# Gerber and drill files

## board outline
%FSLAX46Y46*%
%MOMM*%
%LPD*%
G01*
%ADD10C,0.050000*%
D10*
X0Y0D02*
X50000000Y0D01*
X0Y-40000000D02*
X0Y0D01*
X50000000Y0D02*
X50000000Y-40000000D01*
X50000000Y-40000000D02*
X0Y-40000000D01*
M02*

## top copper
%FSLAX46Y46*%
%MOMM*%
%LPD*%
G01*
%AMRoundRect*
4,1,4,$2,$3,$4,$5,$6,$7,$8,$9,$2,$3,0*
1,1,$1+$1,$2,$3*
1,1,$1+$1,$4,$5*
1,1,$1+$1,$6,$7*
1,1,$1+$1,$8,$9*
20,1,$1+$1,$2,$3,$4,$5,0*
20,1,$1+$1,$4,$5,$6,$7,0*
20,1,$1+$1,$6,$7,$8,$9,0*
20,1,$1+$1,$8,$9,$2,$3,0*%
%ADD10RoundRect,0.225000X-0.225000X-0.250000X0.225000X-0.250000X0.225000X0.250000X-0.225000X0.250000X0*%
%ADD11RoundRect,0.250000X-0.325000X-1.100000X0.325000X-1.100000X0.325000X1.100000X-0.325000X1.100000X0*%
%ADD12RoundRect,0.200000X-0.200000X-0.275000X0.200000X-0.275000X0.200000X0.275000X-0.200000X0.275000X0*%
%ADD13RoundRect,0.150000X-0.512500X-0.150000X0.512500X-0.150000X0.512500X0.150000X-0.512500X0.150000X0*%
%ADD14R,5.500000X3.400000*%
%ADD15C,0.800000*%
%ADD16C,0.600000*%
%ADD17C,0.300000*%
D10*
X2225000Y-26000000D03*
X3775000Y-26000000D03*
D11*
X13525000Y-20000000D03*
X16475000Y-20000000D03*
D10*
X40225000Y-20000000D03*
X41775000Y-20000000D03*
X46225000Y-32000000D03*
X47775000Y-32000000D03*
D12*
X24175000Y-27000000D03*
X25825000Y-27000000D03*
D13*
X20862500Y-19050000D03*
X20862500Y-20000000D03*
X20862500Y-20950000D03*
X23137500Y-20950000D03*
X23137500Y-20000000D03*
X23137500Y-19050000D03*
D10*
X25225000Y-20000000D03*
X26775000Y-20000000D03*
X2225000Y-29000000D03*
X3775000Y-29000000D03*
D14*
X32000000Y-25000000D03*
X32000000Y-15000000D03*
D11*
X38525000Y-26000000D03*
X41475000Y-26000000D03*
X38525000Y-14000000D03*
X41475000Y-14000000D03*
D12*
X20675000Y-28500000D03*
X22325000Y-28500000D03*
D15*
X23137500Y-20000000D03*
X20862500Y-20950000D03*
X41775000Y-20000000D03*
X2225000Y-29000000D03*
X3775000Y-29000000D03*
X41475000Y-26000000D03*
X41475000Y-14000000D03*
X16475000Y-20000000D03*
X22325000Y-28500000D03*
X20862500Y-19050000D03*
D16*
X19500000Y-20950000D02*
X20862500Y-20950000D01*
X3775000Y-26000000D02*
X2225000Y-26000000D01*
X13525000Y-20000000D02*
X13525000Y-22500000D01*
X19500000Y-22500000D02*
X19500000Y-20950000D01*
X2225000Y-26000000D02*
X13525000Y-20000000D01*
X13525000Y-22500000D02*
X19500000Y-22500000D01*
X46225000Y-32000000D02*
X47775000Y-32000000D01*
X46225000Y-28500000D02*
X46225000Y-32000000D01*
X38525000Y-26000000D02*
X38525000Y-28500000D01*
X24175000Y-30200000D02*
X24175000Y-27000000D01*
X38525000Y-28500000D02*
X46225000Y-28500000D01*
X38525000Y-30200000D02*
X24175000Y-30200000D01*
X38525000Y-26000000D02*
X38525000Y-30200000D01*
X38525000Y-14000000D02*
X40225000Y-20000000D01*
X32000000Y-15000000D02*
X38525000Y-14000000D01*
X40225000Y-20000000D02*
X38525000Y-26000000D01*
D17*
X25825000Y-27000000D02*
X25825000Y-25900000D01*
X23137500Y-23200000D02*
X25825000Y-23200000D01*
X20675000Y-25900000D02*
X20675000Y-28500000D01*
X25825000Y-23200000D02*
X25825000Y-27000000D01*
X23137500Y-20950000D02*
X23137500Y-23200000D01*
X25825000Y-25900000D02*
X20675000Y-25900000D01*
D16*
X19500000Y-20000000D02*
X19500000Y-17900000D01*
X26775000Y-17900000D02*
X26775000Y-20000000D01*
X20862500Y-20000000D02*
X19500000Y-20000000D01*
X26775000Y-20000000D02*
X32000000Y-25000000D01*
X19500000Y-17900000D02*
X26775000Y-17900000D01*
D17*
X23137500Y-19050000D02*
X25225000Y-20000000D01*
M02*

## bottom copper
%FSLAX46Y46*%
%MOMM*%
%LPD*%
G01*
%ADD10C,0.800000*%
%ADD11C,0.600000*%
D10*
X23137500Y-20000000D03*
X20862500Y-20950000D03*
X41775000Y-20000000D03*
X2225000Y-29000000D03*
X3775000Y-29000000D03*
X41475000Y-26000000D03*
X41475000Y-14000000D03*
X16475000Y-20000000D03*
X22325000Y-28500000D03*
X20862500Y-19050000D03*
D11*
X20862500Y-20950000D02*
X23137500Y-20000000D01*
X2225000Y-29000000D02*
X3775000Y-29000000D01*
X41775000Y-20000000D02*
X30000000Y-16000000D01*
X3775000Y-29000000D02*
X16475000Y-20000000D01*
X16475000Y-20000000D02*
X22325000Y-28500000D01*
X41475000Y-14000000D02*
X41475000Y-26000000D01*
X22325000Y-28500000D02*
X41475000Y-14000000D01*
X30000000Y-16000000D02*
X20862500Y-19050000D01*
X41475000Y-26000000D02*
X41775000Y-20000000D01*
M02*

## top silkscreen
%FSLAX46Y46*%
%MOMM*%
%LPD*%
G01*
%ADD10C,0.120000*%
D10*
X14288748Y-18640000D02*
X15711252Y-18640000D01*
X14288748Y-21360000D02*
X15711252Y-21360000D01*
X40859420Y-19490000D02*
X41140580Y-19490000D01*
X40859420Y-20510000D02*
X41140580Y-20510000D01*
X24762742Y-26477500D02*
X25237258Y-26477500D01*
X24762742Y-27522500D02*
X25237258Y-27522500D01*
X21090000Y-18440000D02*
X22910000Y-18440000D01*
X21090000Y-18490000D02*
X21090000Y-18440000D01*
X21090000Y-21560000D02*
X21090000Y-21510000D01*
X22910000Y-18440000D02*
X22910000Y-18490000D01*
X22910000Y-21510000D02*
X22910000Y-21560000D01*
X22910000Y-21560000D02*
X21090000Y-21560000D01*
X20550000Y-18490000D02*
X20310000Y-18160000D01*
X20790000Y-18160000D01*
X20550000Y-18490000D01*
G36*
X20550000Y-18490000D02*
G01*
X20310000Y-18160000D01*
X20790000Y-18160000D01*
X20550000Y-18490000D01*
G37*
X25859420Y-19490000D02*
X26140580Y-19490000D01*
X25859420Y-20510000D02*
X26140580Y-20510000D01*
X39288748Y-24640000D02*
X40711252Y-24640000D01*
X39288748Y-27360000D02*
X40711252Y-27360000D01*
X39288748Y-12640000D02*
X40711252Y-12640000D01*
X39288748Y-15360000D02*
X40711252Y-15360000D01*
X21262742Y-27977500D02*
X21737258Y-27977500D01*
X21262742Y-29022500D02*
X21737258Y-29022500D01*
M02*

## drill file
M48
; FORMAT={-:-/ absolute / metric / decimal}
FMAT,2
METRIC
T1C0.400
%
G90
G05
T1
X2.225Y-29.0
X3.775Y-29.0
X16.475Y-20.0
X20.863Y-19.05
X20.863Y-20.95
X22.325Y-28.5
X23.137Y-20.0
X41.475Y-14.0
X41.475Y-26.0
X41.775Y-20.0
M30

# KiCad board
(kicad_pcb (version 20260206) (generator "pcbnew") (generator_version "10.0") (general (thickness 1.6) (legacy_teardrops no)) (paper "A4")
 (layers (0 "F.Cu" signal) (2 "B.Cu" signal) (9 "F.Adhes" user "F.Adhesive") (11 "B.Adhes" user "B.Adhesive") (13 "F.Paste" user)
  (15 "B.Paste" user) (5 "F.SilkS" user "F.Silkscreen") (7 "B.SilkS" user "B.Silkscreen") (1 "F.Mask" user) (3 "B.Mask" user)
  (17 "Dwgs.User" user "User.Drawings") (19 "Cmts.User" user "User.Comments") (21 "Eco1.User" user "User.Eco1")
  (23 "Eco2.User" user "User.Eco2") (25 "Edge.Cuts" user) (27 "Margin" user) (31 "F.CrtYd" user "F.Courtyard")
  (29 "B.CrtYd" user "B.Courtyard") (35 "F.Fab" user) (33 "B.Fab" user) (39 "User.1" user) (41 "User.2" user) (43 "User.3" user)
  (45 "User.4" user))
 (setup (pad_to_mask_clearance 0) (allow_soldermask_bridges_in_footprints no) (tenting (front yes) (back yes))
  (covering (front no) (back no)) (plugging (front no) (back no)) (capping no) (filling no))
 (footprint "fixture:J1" (layer "F.Cu") (at 3 26)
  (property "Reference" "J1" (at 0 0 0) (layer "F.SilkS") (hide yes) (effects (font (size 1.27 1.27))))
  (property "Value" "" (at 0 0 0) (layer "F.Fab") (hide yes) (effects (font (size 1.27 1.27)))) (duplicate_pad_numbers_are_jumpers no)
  (pad "1" smd roundrect (at -0.775 0) (size 0.9 0.95) (layers "F.Cu" "F.Mask" "F.Paste") (roundrect_rratio 0.25) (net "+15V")
   (thermal_bridge_angle 45))
  (pad "2" smd roundrect (at 0.775 0) (size 0.9 0.95) (layers "F.Cu" "F.Mask" "F.Paste") (roundrect_rratio 0.25) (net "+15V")
   (thermal_bridge_angle 45)))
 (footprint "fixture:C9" (layer "F.Cu") (at 15 20)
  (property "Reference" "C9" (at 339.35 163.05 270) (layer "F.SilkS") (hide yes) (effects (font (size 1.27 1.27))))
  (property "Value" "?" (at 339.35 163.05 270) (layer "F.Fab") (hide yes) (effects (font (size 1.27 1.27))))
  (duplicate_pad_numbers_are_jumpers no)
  (fp_line (start -0.711252 -1.36) (end 0.711252 -1.36) (stroke (width 0.12) (type solid)) (layer "F.SilkS"))
  (fp_line (start -0.711252 1.36) (end 0.711252 1.36) (stroke (width 0.12) (type solid)) (layer "F.SilkS"))
  (pad "1" smd roundrect (at -1.475 0) (size 1.15 2.7) (layers "F.Cu" "F.Mask" "F.Paste") (roundrect_rratio 0.217391) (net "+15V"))
  (pad "2" smd roundrect (at 1.475 0) (size 1.15 2.7) (layers "F.Cu" "F.Mask" "F.Paste") (roundrect_rratio 0.217391) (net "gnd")))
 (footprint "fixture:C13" (layer "F.Cu") (at 41 20)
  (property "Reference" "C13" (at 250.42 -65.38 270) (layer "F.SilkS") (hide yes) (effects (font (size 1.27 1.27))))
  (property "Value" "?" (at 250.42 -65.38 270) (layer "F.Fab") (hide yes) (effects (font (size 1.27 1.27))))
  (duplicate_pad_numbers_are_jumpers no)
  (fp_line (start -0.14058 -0.51) (end 0.14058 -0.51) (stroke (width 0.12) (type solid)) (layer "F.SilkS"))
  (fp_line (start -0.14058 0.51) (end 0.14058 0.51) (stroke (width 0.12) (type solid)) (layer "F.SilkS"))
  (pad "1" smd roundrect (at -0.775 0) (size 0.9 0.95) (layers "F.Cu" "F.Mask" "F.Paste") (roundrect_rratio 0.25) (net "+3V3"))
  (pad "2" smd roundrect (at 0.775 0) (size 0.9 0.95) (layers "F.Cu" "F.Mask" "F.Paste") (roundrect_rratio 0.25) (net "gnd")))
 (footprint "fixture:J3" (layer "F.Cu") (at 47 32)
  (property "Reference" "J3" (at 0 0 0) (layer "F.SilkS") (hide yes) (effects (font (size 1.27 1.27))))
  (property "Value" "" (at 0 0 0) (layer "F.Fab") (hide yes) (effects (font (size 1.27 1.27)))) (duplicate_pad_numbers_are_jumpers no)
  (pad "1" smd roundrect (at -0.775 0) (size 0.9 0.95) (layers "F.Cu" "F.Mask" "F.Paste") (roundrect_rratio 0.25) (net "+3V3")
   (thermal_bridge_angle 45))
  (pad "2" smd roundrect (at 0.775 0) (size 0.9 0.95) (layers "F.Cu" "F.Mask" "F.Paste") (roundrect_rratio 0.25) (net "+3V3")
   (thermal_bridge_angle 45)))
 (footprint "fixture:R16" (layer "F.Cu") (at 25 27)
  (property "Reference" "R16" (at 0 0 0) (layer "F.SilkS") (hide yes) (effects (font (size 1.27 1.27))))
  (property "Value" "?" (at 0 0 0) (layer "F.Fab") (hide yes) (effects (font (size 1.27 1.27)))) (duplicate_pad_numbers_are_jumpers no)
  (fp_line (start -0.237258 -0.5225) (end 0.237258 -0.5225) (stroke (width 0.12) (type solid)) (layer "F.SilkS"))
  (fp_line (start -0.237258 0.5225) (end 0.237258 0.5225) (stroke (width 0.12) (type solid)) (layer "F.SilkS"))
  (pad "1" smd roundrect (at -0.825 0) (size 0.8 0.95) (layers "F.Cu" "F.Mask" "F.Paste") (roundrect_rratio 0.25) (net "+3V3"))
  (pad "2" smd roundrect (at 0.825 0) (size 0.8 0.95) (layers "F.Cu" "F.Mask" "F.Paste") (roundrect_rratio 0.25) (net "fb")))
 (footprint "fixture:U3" (layer "F.Cu") (at 22 20)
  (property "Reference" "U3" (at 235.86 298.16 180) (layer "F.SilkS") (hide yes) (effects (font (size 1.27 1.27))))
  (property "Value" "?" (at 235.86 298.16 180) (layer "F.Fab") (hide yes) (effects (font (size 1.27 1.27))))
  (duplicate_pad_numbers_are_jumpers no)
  (fp_line (start -0.91 -1.56) (end 0.91 -1.56) (stroke (width 0.12) (type solid)) (layer "F.SilkS"))
  (fp_line (start -0.91 -1.51) (end -0.91 -1.56) (stroke (width 0.12) (type solid)) (layer "F.SilkS"))
  (fp_line (start -0.91 1.56) (end -0.91 1.51) (stroke (width 0.12) (type solid)) (layer "F.SilkS"))
  (fp_line (start 0.91 -1.56) (end 0.91 -1.51) (stroke (width 0.12) (type solid)) (layer "F.SilkS"))
  (fp_line (start 0.91 1.51) (end 0.91 1.56) (stroke (width 0.12) (type solid)) (layer "F.SilkS"))
  (fp_line (start 0.91 1.56) (end -0.91 1.56) (stroke (width 0.12) (type solid)) (layer "F.SilkS"))
  (fp_poly (pts (xy -1.45 -1.51) (xy -1.69 -1.84) (xy -1.21 -1.84)) (stroke (width 0.12) (type solid)) (fill yes) (layer "F.SilkS"))
  (pad "1" smd roundrect (at -1.1375 -0.95) (size 1.325 0.6) (layers "F.Cu" "F.Mask" "F.Paste") (roundrect_rratio 0.25) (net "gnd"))
  (pad "2" smd roundrect (at -1.1375 0) (size 1.325 0.6) (layers "F.Cu" "F.Mask" "F.Paste") (roundrect_rratio 0.25) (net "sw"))
  (pad "3" smd roundrect (at -1.1375 0.95) (size 1.325 0.6) (layers "F.Cu" "F.Mask" "F.Paste") (roundrect_rratio 0.25) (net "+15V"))
  (pad "4" smd roundrect (at 1.1375 0.95) (size 1.325 0.6) (layers "F.Cu" "F.Mask" "F.Paste") (roundrect_rratio 0.25) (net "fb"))
  (pad "5" smd roundrect (at 1.1375 0) (size 1.325 0.6) (layers "F.Cu" "F.Mask" "F.Paste") (roundrect_rratio 0.25) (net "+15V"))
  (pad "6" smd roundrect (at 1.1375 -0.95) (size 1.325 0.6) (layers "F.Cu" "F.Mask" "F.Paste") (roundrect_rratio 0.25) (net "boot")))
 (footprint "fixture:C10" (layer "F.Cu") (at 26 20)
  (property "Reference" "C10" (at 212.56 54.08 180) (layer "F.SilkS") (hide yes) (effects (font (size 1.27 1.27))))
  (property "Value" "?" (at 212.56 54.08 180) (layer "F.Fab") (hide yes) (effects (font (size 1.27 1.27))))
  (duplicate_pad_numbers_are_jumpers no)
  (fp_line (start -0.14058 -0.51) (end 0.14058 -0.51) (stroke (width 0.12) (type solid)) (layer "F.SilkS"))
  (fp_line (start -0.14058 0.51) (end 0.14058 0.51) (stroke (width 0.12) (type solid)) (layer "F.SilkS"))
  (pad "1" smd roundrect (at -0.775 0) (size 0.9 0.95) (layers "F.Cu" "F.Mask" "F.Paste") (roundrect_rratio 0.25) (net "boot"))
  (pad "2" smd roundrect (at 0.775 0) (size 0.9 0.95) (layers "F.Cu" "F.Mask" "F.Paste") (roundrect_rratio 0.25) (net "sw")))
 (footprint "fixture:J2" (layer "F.Cu") (at 3 29)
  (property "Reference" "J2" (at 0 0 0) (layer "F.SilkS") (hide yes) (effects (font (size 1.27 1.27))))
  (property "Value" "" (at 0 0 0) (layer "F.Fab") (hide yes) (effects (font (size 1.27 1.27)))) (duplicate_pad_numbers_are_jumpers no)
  (pad "1" smd roundrect (at -0.775 0) (size 0.9 0.95) (layers "F.Cu" "F.Mask" "F.Paste") (roundrect_rratio 0.25) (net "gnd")
   (thermal_bridge_angle 45))
  (pad "2" smd roundrect (at 0.775 0) (size 0.9 0.95) (layers "F.Cu" "F.Mask" "F.Paste") (roundrect_rratio 0.25) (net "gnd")
   (thermal_bridge_angle 45)))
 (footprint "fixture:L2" (layer "F.Cu") (at 32 20 90)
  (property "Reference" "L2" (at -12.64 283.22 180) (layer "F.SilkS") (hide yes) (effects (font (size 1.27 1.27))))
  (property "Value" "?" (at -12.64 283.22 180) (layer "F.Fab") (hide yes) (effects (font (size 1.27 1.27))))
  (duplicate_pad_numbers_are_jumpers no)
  (pad "1" smd rect (at -5 0 90) (size 3.4 5.5) (layers "F.Cu" "F.Mask" "F.Paste") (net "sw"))
  (pad "2" smd rect (at 5 0 90) (size 3.4 5.5) (layers "F.Cu" "F.Mask" "F.Paste") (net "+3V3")))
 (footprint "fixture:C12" (layer "F.Cu") (at 40 26)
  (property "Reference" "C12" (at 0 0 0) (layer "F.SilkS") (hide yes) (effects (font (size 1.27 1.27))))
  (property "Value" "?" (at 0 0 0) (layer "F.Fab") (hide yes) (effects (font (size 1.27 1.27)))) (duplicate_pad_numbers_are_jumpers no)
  (fp_line (start -0.711252 -1.36) (end 0.711252 -1.36) (stroke (width 0.12) (type solid)) (layer "F.SilkS"))
  (fp_line (start -0.711252 1.36) (end 0.711252 1.36) (stroke (width 0.12) (type solid)) (layer "F.SilkS"))
  (pad "1" smd roundrect (at -1.475 0) (size 1.15 2.7) (layers "F.Cu" "F.Mask" "F.Paste") (roundrect_rratio 0.217391) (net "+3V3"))
  (pad "2" smd roundrect (at 1.475 0) (size 1.15 2.7) (layers "F.Cu" "F.Mask" "F.Paste") (roundrect_rratio 0.217391) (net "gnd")))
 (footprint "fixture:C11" (layer "F.Cu") (at 40 14)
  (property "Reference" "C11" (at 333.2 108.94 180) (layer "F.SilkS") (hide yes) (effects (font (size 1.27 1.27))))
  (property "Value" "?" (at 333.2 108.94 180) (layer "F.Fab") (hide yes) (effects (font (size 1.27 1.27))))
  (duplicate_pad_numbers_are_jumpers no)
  (fp_line (start -0.711252 -1.36) (end 0.711252 -1.36) (stroke (width 0.12) (type solid)) (layer "F.SilkS"))
  (fp_line (start -0.711252 1.36) (end 0.711252 1.36) (stroke (width 0.12) (type solid)) (layer "F.SilkS"))
  (pad "1" smd roundrect (at -1.475 0) (size 1.15 2.7) (layers "F.Cu" "F.Mask" "F.Paste") (roundrect_rratio 0.217391) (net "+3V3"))
  (pad "2" smd roundrect (at 1.475 0) (size 1.15 2.7) (layers "F.Cu" "F.Mask" "F.Paste") (roundrect_rratio 0.217391) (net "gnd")))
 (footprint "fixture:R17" (layer "F.Cu") (at 21.5 28.5)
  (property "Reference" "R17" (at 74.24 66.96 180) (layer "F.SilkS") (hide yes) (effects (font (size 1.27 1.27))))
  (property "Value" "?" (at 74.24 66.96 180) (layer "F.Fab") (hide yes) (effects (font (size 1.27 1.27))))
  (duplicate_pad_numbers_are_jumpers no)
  (fp_line (start -0.237258 -0.5225) (end 0.237258 -0.5225) (stroke (width 0.12) (type solid)) (layer "F.SilkS"))
  (fp_line (start -0.237258 0.5225) (end 0.237258 0.5225) (stroke (width 0.12) (type solid)) (layer "F.SilkS"))
  (pad "1" smd roundrect (at -0.825 0) (size 0.8 0.95) (layers "F.Cu" "F.Mask" "F.Paste") (roundrect_rratio 0.25) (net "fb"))
  (pad "2" smd roundrect (at 0.825 0) (size 0.8 0.95) (layers "F.Cu" "F.Mask" "F.Paste") (roundrect_rratio 0.25) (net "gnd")))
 (gr_line (start 0 0) (end 50 0) (stroke (width 0.05) (type default)) (layer "Edge.Cuts"))
 (gr_line (start 0 40) (end 0 0) (stroke (width 0.05) (type default)) (layer "Edge.Cuts"))
 (gr_line (start 50 0) (end 50 40) (stroke (width 0.05) (type default)) (layer "Edge.Cuts"))
 (gr_line (start 50 40) (end 0 40) (stroke (width 0.05) (type default)) (layer "Edge.Cuts"))
 (segment (start 19.5 20.95) (end 20.8625 20.95) (width 0.6) (layer "F.Cu") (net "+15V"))
 (segment (start 3.775 26) (end 2.225 26) (width 0.6) (layer "F.Cu") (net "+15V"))
 (segment (start 13.525 20) (end 13.525 22.5) (width 0.6) (layer "F.Cu") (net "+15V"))
 (segment (start 19.5 22.5) (end 19.5 20.95) (width 0.6) (layer "F.Cu") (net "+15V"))
 (segment (start 2.225 26) (end 13.525 20) (width 0.6) (layer "F.Cu") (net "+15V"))
 (segment (start 13.525 22.5) (end 19.5 22.5) (width 0.6) (layer "F.Cu") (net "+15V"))
 (via (at 23.1375 20) (size 0.8) (drill 0.4) (layers "F.Cu" "B.Cu") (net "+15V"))
 (via (at 20.8625 20.95) (size 0.8) (drill 0.4) (layers "F.Cu" "B.Cu") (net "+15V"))
 (segment (start 20.8625 20.95) (end 23.1375 20) (width 0.6) (layer "B.Cu") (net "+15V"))
 (via (at 41.775 20) (size 0.8) (drill 0.4) (layers "F.Cu" "B.Cu") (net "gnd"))
 (via (at 2.225 29) (size 0.8) (drill 0.4) (layers "F.Cu" "B.Cu") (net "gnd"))
 (via (at 3.775 29) (size 0.8) (drill 0.4) (layers "F.Cu" "B.Cu") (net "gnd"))
 (via (at 41.475 26) (size 0.8) (drill 0.4) (layers "F.Cu" "B.Cu") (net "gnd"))
 (via (at 41.475 14) (size 0.8) (drill 0.4) (layers "F.Cu" "B.Cu") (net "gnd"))
 (via (at 16.475 20) (size 0.8) (drill 0.4) (layers "F.Cu" "B.Cu") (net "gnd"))
 (via (at 22.325 28.5) (size 0.8) (drill 0.4) (layers "F.Cu" "B.Cu") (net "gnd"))
 (via (at 20.8625 19.05) (size 0.8) (drill 0.4) (layers "F.Cu" "B.Cu") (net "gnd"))
 (segment (start 2.225 29) (end 3.775 29) (width 0.6) (layer "B.Cu") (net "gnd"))
 (segment (start 41.775 20) (end 30 16) (width 0.6) (layer "B.Cu") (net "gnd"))
 (segment (start 3.775 29) (end 16.475 20) (width 0.6) (layer "B.Cu") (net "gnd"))
 (segment (start 16.475 20) (end 22.325 28.5) (width 0.6) (layer "B.Cu") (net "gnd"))
 (segment (start 41.475 14) (end 41.475 26) (width 0.6) (layer "B.Cu") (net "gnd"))
 (segment (start 22.325 28.5) (end 41.475 14) (width 0.6) (layer "B.Cu") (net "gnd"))
 (segment (start 30 16) (end 20.8625 19.05) (width 0.6) (layer "B.Cu") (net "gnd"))
 (segment (start 41.475 26) (end 41.775 20) (width 0.6) (layer "B.Cu") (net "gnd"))
 (segment (start 46.225 32) (end 47.775 32) (width 0.6) (layer "F.Cu") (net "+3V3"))
 (segment (start 46.225 28.5) (end 46.225 32) (width 0.6) (layer "F.Cu") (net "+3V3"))
 (segment (start 38.525 26) (end 38.525 28.5) (width 0.6) (layer "F.Cu") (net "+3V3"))
 (segment (start 24.175 30.2) (end 24.175 27) (width 0.6) (layer "F.Cu") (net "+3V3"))
 (segment (start 38.525 28.5) (end 46.225 28.5) (width 0.6) (layer "F.Cu") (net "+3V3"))
 (segment (start 38.525 30.2) (end 24.175 30.2) (width 0.6) (layer "F.Cu") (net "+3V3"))
 (segment (start 38.525 26) (end 38.525 30.2) (width 0.6) (layer "F.Cu") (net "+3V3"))
 (segment (start 38.525 14) (end 40.225 20) (width 0.6) (layer "F.Cu") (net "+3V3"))
 (segment (start 32 15) (end 38.525 14) (width 0.6) (layer "F.Cu") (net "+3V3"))
 (segment (start 40.225 20) (end 38.525 26) (width 0.6) (layer "F.Cu") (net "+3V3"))
 (segment (start 25.825 27) (end 25.825 25.9) (width 0.3) (layer "F.Cu") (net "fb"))
 (segment (start 23.1375 23.2) (end 25.825 23.2) (width 0.3) (layer "F.Cu") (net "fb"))
 (segment (start 20.675 25.9) (end 20.675 28.5) (width 0.3) (layer "F.Cu") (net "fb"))
 (segment (start 25.825 23.2) (end 25.825 27) (width 0.3) (layer "F.Cu") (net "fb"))
 (segment (start 23.1375 20.95) (end 23.1375 23.2) (width 0.3) (layer "F.Cu") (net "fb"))
 (segment (start 25.825 25.9) (end 20.675 25.9) (width 0.3) (layer "F.Cu") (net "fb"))
 (segment (start 19.5 20) (end 19.5 17.9) (width 0.6) (layer "F.Cu") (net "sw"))
 (segment (start 26.775 17.9) (end 26.775 20) (width 0.6) (layer "F.Cu") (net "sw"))
 (segment (start 20.8625 20) (end 19.5 20) (width 0.6) (layer "F.Cu") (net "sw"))
 (segment (start 26.775 20) (end 32 25) (width 0.6) (layer "F.Cu") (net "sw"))
 (segment (start 19.5 17.9) (end 26.775 17.9) (width 0.6) (layer "F.Cu") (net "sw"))
 (segment (start 23.1375 19.05) (end 25.225 20) (width 0.3) (layer "F.Cu") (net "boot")))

